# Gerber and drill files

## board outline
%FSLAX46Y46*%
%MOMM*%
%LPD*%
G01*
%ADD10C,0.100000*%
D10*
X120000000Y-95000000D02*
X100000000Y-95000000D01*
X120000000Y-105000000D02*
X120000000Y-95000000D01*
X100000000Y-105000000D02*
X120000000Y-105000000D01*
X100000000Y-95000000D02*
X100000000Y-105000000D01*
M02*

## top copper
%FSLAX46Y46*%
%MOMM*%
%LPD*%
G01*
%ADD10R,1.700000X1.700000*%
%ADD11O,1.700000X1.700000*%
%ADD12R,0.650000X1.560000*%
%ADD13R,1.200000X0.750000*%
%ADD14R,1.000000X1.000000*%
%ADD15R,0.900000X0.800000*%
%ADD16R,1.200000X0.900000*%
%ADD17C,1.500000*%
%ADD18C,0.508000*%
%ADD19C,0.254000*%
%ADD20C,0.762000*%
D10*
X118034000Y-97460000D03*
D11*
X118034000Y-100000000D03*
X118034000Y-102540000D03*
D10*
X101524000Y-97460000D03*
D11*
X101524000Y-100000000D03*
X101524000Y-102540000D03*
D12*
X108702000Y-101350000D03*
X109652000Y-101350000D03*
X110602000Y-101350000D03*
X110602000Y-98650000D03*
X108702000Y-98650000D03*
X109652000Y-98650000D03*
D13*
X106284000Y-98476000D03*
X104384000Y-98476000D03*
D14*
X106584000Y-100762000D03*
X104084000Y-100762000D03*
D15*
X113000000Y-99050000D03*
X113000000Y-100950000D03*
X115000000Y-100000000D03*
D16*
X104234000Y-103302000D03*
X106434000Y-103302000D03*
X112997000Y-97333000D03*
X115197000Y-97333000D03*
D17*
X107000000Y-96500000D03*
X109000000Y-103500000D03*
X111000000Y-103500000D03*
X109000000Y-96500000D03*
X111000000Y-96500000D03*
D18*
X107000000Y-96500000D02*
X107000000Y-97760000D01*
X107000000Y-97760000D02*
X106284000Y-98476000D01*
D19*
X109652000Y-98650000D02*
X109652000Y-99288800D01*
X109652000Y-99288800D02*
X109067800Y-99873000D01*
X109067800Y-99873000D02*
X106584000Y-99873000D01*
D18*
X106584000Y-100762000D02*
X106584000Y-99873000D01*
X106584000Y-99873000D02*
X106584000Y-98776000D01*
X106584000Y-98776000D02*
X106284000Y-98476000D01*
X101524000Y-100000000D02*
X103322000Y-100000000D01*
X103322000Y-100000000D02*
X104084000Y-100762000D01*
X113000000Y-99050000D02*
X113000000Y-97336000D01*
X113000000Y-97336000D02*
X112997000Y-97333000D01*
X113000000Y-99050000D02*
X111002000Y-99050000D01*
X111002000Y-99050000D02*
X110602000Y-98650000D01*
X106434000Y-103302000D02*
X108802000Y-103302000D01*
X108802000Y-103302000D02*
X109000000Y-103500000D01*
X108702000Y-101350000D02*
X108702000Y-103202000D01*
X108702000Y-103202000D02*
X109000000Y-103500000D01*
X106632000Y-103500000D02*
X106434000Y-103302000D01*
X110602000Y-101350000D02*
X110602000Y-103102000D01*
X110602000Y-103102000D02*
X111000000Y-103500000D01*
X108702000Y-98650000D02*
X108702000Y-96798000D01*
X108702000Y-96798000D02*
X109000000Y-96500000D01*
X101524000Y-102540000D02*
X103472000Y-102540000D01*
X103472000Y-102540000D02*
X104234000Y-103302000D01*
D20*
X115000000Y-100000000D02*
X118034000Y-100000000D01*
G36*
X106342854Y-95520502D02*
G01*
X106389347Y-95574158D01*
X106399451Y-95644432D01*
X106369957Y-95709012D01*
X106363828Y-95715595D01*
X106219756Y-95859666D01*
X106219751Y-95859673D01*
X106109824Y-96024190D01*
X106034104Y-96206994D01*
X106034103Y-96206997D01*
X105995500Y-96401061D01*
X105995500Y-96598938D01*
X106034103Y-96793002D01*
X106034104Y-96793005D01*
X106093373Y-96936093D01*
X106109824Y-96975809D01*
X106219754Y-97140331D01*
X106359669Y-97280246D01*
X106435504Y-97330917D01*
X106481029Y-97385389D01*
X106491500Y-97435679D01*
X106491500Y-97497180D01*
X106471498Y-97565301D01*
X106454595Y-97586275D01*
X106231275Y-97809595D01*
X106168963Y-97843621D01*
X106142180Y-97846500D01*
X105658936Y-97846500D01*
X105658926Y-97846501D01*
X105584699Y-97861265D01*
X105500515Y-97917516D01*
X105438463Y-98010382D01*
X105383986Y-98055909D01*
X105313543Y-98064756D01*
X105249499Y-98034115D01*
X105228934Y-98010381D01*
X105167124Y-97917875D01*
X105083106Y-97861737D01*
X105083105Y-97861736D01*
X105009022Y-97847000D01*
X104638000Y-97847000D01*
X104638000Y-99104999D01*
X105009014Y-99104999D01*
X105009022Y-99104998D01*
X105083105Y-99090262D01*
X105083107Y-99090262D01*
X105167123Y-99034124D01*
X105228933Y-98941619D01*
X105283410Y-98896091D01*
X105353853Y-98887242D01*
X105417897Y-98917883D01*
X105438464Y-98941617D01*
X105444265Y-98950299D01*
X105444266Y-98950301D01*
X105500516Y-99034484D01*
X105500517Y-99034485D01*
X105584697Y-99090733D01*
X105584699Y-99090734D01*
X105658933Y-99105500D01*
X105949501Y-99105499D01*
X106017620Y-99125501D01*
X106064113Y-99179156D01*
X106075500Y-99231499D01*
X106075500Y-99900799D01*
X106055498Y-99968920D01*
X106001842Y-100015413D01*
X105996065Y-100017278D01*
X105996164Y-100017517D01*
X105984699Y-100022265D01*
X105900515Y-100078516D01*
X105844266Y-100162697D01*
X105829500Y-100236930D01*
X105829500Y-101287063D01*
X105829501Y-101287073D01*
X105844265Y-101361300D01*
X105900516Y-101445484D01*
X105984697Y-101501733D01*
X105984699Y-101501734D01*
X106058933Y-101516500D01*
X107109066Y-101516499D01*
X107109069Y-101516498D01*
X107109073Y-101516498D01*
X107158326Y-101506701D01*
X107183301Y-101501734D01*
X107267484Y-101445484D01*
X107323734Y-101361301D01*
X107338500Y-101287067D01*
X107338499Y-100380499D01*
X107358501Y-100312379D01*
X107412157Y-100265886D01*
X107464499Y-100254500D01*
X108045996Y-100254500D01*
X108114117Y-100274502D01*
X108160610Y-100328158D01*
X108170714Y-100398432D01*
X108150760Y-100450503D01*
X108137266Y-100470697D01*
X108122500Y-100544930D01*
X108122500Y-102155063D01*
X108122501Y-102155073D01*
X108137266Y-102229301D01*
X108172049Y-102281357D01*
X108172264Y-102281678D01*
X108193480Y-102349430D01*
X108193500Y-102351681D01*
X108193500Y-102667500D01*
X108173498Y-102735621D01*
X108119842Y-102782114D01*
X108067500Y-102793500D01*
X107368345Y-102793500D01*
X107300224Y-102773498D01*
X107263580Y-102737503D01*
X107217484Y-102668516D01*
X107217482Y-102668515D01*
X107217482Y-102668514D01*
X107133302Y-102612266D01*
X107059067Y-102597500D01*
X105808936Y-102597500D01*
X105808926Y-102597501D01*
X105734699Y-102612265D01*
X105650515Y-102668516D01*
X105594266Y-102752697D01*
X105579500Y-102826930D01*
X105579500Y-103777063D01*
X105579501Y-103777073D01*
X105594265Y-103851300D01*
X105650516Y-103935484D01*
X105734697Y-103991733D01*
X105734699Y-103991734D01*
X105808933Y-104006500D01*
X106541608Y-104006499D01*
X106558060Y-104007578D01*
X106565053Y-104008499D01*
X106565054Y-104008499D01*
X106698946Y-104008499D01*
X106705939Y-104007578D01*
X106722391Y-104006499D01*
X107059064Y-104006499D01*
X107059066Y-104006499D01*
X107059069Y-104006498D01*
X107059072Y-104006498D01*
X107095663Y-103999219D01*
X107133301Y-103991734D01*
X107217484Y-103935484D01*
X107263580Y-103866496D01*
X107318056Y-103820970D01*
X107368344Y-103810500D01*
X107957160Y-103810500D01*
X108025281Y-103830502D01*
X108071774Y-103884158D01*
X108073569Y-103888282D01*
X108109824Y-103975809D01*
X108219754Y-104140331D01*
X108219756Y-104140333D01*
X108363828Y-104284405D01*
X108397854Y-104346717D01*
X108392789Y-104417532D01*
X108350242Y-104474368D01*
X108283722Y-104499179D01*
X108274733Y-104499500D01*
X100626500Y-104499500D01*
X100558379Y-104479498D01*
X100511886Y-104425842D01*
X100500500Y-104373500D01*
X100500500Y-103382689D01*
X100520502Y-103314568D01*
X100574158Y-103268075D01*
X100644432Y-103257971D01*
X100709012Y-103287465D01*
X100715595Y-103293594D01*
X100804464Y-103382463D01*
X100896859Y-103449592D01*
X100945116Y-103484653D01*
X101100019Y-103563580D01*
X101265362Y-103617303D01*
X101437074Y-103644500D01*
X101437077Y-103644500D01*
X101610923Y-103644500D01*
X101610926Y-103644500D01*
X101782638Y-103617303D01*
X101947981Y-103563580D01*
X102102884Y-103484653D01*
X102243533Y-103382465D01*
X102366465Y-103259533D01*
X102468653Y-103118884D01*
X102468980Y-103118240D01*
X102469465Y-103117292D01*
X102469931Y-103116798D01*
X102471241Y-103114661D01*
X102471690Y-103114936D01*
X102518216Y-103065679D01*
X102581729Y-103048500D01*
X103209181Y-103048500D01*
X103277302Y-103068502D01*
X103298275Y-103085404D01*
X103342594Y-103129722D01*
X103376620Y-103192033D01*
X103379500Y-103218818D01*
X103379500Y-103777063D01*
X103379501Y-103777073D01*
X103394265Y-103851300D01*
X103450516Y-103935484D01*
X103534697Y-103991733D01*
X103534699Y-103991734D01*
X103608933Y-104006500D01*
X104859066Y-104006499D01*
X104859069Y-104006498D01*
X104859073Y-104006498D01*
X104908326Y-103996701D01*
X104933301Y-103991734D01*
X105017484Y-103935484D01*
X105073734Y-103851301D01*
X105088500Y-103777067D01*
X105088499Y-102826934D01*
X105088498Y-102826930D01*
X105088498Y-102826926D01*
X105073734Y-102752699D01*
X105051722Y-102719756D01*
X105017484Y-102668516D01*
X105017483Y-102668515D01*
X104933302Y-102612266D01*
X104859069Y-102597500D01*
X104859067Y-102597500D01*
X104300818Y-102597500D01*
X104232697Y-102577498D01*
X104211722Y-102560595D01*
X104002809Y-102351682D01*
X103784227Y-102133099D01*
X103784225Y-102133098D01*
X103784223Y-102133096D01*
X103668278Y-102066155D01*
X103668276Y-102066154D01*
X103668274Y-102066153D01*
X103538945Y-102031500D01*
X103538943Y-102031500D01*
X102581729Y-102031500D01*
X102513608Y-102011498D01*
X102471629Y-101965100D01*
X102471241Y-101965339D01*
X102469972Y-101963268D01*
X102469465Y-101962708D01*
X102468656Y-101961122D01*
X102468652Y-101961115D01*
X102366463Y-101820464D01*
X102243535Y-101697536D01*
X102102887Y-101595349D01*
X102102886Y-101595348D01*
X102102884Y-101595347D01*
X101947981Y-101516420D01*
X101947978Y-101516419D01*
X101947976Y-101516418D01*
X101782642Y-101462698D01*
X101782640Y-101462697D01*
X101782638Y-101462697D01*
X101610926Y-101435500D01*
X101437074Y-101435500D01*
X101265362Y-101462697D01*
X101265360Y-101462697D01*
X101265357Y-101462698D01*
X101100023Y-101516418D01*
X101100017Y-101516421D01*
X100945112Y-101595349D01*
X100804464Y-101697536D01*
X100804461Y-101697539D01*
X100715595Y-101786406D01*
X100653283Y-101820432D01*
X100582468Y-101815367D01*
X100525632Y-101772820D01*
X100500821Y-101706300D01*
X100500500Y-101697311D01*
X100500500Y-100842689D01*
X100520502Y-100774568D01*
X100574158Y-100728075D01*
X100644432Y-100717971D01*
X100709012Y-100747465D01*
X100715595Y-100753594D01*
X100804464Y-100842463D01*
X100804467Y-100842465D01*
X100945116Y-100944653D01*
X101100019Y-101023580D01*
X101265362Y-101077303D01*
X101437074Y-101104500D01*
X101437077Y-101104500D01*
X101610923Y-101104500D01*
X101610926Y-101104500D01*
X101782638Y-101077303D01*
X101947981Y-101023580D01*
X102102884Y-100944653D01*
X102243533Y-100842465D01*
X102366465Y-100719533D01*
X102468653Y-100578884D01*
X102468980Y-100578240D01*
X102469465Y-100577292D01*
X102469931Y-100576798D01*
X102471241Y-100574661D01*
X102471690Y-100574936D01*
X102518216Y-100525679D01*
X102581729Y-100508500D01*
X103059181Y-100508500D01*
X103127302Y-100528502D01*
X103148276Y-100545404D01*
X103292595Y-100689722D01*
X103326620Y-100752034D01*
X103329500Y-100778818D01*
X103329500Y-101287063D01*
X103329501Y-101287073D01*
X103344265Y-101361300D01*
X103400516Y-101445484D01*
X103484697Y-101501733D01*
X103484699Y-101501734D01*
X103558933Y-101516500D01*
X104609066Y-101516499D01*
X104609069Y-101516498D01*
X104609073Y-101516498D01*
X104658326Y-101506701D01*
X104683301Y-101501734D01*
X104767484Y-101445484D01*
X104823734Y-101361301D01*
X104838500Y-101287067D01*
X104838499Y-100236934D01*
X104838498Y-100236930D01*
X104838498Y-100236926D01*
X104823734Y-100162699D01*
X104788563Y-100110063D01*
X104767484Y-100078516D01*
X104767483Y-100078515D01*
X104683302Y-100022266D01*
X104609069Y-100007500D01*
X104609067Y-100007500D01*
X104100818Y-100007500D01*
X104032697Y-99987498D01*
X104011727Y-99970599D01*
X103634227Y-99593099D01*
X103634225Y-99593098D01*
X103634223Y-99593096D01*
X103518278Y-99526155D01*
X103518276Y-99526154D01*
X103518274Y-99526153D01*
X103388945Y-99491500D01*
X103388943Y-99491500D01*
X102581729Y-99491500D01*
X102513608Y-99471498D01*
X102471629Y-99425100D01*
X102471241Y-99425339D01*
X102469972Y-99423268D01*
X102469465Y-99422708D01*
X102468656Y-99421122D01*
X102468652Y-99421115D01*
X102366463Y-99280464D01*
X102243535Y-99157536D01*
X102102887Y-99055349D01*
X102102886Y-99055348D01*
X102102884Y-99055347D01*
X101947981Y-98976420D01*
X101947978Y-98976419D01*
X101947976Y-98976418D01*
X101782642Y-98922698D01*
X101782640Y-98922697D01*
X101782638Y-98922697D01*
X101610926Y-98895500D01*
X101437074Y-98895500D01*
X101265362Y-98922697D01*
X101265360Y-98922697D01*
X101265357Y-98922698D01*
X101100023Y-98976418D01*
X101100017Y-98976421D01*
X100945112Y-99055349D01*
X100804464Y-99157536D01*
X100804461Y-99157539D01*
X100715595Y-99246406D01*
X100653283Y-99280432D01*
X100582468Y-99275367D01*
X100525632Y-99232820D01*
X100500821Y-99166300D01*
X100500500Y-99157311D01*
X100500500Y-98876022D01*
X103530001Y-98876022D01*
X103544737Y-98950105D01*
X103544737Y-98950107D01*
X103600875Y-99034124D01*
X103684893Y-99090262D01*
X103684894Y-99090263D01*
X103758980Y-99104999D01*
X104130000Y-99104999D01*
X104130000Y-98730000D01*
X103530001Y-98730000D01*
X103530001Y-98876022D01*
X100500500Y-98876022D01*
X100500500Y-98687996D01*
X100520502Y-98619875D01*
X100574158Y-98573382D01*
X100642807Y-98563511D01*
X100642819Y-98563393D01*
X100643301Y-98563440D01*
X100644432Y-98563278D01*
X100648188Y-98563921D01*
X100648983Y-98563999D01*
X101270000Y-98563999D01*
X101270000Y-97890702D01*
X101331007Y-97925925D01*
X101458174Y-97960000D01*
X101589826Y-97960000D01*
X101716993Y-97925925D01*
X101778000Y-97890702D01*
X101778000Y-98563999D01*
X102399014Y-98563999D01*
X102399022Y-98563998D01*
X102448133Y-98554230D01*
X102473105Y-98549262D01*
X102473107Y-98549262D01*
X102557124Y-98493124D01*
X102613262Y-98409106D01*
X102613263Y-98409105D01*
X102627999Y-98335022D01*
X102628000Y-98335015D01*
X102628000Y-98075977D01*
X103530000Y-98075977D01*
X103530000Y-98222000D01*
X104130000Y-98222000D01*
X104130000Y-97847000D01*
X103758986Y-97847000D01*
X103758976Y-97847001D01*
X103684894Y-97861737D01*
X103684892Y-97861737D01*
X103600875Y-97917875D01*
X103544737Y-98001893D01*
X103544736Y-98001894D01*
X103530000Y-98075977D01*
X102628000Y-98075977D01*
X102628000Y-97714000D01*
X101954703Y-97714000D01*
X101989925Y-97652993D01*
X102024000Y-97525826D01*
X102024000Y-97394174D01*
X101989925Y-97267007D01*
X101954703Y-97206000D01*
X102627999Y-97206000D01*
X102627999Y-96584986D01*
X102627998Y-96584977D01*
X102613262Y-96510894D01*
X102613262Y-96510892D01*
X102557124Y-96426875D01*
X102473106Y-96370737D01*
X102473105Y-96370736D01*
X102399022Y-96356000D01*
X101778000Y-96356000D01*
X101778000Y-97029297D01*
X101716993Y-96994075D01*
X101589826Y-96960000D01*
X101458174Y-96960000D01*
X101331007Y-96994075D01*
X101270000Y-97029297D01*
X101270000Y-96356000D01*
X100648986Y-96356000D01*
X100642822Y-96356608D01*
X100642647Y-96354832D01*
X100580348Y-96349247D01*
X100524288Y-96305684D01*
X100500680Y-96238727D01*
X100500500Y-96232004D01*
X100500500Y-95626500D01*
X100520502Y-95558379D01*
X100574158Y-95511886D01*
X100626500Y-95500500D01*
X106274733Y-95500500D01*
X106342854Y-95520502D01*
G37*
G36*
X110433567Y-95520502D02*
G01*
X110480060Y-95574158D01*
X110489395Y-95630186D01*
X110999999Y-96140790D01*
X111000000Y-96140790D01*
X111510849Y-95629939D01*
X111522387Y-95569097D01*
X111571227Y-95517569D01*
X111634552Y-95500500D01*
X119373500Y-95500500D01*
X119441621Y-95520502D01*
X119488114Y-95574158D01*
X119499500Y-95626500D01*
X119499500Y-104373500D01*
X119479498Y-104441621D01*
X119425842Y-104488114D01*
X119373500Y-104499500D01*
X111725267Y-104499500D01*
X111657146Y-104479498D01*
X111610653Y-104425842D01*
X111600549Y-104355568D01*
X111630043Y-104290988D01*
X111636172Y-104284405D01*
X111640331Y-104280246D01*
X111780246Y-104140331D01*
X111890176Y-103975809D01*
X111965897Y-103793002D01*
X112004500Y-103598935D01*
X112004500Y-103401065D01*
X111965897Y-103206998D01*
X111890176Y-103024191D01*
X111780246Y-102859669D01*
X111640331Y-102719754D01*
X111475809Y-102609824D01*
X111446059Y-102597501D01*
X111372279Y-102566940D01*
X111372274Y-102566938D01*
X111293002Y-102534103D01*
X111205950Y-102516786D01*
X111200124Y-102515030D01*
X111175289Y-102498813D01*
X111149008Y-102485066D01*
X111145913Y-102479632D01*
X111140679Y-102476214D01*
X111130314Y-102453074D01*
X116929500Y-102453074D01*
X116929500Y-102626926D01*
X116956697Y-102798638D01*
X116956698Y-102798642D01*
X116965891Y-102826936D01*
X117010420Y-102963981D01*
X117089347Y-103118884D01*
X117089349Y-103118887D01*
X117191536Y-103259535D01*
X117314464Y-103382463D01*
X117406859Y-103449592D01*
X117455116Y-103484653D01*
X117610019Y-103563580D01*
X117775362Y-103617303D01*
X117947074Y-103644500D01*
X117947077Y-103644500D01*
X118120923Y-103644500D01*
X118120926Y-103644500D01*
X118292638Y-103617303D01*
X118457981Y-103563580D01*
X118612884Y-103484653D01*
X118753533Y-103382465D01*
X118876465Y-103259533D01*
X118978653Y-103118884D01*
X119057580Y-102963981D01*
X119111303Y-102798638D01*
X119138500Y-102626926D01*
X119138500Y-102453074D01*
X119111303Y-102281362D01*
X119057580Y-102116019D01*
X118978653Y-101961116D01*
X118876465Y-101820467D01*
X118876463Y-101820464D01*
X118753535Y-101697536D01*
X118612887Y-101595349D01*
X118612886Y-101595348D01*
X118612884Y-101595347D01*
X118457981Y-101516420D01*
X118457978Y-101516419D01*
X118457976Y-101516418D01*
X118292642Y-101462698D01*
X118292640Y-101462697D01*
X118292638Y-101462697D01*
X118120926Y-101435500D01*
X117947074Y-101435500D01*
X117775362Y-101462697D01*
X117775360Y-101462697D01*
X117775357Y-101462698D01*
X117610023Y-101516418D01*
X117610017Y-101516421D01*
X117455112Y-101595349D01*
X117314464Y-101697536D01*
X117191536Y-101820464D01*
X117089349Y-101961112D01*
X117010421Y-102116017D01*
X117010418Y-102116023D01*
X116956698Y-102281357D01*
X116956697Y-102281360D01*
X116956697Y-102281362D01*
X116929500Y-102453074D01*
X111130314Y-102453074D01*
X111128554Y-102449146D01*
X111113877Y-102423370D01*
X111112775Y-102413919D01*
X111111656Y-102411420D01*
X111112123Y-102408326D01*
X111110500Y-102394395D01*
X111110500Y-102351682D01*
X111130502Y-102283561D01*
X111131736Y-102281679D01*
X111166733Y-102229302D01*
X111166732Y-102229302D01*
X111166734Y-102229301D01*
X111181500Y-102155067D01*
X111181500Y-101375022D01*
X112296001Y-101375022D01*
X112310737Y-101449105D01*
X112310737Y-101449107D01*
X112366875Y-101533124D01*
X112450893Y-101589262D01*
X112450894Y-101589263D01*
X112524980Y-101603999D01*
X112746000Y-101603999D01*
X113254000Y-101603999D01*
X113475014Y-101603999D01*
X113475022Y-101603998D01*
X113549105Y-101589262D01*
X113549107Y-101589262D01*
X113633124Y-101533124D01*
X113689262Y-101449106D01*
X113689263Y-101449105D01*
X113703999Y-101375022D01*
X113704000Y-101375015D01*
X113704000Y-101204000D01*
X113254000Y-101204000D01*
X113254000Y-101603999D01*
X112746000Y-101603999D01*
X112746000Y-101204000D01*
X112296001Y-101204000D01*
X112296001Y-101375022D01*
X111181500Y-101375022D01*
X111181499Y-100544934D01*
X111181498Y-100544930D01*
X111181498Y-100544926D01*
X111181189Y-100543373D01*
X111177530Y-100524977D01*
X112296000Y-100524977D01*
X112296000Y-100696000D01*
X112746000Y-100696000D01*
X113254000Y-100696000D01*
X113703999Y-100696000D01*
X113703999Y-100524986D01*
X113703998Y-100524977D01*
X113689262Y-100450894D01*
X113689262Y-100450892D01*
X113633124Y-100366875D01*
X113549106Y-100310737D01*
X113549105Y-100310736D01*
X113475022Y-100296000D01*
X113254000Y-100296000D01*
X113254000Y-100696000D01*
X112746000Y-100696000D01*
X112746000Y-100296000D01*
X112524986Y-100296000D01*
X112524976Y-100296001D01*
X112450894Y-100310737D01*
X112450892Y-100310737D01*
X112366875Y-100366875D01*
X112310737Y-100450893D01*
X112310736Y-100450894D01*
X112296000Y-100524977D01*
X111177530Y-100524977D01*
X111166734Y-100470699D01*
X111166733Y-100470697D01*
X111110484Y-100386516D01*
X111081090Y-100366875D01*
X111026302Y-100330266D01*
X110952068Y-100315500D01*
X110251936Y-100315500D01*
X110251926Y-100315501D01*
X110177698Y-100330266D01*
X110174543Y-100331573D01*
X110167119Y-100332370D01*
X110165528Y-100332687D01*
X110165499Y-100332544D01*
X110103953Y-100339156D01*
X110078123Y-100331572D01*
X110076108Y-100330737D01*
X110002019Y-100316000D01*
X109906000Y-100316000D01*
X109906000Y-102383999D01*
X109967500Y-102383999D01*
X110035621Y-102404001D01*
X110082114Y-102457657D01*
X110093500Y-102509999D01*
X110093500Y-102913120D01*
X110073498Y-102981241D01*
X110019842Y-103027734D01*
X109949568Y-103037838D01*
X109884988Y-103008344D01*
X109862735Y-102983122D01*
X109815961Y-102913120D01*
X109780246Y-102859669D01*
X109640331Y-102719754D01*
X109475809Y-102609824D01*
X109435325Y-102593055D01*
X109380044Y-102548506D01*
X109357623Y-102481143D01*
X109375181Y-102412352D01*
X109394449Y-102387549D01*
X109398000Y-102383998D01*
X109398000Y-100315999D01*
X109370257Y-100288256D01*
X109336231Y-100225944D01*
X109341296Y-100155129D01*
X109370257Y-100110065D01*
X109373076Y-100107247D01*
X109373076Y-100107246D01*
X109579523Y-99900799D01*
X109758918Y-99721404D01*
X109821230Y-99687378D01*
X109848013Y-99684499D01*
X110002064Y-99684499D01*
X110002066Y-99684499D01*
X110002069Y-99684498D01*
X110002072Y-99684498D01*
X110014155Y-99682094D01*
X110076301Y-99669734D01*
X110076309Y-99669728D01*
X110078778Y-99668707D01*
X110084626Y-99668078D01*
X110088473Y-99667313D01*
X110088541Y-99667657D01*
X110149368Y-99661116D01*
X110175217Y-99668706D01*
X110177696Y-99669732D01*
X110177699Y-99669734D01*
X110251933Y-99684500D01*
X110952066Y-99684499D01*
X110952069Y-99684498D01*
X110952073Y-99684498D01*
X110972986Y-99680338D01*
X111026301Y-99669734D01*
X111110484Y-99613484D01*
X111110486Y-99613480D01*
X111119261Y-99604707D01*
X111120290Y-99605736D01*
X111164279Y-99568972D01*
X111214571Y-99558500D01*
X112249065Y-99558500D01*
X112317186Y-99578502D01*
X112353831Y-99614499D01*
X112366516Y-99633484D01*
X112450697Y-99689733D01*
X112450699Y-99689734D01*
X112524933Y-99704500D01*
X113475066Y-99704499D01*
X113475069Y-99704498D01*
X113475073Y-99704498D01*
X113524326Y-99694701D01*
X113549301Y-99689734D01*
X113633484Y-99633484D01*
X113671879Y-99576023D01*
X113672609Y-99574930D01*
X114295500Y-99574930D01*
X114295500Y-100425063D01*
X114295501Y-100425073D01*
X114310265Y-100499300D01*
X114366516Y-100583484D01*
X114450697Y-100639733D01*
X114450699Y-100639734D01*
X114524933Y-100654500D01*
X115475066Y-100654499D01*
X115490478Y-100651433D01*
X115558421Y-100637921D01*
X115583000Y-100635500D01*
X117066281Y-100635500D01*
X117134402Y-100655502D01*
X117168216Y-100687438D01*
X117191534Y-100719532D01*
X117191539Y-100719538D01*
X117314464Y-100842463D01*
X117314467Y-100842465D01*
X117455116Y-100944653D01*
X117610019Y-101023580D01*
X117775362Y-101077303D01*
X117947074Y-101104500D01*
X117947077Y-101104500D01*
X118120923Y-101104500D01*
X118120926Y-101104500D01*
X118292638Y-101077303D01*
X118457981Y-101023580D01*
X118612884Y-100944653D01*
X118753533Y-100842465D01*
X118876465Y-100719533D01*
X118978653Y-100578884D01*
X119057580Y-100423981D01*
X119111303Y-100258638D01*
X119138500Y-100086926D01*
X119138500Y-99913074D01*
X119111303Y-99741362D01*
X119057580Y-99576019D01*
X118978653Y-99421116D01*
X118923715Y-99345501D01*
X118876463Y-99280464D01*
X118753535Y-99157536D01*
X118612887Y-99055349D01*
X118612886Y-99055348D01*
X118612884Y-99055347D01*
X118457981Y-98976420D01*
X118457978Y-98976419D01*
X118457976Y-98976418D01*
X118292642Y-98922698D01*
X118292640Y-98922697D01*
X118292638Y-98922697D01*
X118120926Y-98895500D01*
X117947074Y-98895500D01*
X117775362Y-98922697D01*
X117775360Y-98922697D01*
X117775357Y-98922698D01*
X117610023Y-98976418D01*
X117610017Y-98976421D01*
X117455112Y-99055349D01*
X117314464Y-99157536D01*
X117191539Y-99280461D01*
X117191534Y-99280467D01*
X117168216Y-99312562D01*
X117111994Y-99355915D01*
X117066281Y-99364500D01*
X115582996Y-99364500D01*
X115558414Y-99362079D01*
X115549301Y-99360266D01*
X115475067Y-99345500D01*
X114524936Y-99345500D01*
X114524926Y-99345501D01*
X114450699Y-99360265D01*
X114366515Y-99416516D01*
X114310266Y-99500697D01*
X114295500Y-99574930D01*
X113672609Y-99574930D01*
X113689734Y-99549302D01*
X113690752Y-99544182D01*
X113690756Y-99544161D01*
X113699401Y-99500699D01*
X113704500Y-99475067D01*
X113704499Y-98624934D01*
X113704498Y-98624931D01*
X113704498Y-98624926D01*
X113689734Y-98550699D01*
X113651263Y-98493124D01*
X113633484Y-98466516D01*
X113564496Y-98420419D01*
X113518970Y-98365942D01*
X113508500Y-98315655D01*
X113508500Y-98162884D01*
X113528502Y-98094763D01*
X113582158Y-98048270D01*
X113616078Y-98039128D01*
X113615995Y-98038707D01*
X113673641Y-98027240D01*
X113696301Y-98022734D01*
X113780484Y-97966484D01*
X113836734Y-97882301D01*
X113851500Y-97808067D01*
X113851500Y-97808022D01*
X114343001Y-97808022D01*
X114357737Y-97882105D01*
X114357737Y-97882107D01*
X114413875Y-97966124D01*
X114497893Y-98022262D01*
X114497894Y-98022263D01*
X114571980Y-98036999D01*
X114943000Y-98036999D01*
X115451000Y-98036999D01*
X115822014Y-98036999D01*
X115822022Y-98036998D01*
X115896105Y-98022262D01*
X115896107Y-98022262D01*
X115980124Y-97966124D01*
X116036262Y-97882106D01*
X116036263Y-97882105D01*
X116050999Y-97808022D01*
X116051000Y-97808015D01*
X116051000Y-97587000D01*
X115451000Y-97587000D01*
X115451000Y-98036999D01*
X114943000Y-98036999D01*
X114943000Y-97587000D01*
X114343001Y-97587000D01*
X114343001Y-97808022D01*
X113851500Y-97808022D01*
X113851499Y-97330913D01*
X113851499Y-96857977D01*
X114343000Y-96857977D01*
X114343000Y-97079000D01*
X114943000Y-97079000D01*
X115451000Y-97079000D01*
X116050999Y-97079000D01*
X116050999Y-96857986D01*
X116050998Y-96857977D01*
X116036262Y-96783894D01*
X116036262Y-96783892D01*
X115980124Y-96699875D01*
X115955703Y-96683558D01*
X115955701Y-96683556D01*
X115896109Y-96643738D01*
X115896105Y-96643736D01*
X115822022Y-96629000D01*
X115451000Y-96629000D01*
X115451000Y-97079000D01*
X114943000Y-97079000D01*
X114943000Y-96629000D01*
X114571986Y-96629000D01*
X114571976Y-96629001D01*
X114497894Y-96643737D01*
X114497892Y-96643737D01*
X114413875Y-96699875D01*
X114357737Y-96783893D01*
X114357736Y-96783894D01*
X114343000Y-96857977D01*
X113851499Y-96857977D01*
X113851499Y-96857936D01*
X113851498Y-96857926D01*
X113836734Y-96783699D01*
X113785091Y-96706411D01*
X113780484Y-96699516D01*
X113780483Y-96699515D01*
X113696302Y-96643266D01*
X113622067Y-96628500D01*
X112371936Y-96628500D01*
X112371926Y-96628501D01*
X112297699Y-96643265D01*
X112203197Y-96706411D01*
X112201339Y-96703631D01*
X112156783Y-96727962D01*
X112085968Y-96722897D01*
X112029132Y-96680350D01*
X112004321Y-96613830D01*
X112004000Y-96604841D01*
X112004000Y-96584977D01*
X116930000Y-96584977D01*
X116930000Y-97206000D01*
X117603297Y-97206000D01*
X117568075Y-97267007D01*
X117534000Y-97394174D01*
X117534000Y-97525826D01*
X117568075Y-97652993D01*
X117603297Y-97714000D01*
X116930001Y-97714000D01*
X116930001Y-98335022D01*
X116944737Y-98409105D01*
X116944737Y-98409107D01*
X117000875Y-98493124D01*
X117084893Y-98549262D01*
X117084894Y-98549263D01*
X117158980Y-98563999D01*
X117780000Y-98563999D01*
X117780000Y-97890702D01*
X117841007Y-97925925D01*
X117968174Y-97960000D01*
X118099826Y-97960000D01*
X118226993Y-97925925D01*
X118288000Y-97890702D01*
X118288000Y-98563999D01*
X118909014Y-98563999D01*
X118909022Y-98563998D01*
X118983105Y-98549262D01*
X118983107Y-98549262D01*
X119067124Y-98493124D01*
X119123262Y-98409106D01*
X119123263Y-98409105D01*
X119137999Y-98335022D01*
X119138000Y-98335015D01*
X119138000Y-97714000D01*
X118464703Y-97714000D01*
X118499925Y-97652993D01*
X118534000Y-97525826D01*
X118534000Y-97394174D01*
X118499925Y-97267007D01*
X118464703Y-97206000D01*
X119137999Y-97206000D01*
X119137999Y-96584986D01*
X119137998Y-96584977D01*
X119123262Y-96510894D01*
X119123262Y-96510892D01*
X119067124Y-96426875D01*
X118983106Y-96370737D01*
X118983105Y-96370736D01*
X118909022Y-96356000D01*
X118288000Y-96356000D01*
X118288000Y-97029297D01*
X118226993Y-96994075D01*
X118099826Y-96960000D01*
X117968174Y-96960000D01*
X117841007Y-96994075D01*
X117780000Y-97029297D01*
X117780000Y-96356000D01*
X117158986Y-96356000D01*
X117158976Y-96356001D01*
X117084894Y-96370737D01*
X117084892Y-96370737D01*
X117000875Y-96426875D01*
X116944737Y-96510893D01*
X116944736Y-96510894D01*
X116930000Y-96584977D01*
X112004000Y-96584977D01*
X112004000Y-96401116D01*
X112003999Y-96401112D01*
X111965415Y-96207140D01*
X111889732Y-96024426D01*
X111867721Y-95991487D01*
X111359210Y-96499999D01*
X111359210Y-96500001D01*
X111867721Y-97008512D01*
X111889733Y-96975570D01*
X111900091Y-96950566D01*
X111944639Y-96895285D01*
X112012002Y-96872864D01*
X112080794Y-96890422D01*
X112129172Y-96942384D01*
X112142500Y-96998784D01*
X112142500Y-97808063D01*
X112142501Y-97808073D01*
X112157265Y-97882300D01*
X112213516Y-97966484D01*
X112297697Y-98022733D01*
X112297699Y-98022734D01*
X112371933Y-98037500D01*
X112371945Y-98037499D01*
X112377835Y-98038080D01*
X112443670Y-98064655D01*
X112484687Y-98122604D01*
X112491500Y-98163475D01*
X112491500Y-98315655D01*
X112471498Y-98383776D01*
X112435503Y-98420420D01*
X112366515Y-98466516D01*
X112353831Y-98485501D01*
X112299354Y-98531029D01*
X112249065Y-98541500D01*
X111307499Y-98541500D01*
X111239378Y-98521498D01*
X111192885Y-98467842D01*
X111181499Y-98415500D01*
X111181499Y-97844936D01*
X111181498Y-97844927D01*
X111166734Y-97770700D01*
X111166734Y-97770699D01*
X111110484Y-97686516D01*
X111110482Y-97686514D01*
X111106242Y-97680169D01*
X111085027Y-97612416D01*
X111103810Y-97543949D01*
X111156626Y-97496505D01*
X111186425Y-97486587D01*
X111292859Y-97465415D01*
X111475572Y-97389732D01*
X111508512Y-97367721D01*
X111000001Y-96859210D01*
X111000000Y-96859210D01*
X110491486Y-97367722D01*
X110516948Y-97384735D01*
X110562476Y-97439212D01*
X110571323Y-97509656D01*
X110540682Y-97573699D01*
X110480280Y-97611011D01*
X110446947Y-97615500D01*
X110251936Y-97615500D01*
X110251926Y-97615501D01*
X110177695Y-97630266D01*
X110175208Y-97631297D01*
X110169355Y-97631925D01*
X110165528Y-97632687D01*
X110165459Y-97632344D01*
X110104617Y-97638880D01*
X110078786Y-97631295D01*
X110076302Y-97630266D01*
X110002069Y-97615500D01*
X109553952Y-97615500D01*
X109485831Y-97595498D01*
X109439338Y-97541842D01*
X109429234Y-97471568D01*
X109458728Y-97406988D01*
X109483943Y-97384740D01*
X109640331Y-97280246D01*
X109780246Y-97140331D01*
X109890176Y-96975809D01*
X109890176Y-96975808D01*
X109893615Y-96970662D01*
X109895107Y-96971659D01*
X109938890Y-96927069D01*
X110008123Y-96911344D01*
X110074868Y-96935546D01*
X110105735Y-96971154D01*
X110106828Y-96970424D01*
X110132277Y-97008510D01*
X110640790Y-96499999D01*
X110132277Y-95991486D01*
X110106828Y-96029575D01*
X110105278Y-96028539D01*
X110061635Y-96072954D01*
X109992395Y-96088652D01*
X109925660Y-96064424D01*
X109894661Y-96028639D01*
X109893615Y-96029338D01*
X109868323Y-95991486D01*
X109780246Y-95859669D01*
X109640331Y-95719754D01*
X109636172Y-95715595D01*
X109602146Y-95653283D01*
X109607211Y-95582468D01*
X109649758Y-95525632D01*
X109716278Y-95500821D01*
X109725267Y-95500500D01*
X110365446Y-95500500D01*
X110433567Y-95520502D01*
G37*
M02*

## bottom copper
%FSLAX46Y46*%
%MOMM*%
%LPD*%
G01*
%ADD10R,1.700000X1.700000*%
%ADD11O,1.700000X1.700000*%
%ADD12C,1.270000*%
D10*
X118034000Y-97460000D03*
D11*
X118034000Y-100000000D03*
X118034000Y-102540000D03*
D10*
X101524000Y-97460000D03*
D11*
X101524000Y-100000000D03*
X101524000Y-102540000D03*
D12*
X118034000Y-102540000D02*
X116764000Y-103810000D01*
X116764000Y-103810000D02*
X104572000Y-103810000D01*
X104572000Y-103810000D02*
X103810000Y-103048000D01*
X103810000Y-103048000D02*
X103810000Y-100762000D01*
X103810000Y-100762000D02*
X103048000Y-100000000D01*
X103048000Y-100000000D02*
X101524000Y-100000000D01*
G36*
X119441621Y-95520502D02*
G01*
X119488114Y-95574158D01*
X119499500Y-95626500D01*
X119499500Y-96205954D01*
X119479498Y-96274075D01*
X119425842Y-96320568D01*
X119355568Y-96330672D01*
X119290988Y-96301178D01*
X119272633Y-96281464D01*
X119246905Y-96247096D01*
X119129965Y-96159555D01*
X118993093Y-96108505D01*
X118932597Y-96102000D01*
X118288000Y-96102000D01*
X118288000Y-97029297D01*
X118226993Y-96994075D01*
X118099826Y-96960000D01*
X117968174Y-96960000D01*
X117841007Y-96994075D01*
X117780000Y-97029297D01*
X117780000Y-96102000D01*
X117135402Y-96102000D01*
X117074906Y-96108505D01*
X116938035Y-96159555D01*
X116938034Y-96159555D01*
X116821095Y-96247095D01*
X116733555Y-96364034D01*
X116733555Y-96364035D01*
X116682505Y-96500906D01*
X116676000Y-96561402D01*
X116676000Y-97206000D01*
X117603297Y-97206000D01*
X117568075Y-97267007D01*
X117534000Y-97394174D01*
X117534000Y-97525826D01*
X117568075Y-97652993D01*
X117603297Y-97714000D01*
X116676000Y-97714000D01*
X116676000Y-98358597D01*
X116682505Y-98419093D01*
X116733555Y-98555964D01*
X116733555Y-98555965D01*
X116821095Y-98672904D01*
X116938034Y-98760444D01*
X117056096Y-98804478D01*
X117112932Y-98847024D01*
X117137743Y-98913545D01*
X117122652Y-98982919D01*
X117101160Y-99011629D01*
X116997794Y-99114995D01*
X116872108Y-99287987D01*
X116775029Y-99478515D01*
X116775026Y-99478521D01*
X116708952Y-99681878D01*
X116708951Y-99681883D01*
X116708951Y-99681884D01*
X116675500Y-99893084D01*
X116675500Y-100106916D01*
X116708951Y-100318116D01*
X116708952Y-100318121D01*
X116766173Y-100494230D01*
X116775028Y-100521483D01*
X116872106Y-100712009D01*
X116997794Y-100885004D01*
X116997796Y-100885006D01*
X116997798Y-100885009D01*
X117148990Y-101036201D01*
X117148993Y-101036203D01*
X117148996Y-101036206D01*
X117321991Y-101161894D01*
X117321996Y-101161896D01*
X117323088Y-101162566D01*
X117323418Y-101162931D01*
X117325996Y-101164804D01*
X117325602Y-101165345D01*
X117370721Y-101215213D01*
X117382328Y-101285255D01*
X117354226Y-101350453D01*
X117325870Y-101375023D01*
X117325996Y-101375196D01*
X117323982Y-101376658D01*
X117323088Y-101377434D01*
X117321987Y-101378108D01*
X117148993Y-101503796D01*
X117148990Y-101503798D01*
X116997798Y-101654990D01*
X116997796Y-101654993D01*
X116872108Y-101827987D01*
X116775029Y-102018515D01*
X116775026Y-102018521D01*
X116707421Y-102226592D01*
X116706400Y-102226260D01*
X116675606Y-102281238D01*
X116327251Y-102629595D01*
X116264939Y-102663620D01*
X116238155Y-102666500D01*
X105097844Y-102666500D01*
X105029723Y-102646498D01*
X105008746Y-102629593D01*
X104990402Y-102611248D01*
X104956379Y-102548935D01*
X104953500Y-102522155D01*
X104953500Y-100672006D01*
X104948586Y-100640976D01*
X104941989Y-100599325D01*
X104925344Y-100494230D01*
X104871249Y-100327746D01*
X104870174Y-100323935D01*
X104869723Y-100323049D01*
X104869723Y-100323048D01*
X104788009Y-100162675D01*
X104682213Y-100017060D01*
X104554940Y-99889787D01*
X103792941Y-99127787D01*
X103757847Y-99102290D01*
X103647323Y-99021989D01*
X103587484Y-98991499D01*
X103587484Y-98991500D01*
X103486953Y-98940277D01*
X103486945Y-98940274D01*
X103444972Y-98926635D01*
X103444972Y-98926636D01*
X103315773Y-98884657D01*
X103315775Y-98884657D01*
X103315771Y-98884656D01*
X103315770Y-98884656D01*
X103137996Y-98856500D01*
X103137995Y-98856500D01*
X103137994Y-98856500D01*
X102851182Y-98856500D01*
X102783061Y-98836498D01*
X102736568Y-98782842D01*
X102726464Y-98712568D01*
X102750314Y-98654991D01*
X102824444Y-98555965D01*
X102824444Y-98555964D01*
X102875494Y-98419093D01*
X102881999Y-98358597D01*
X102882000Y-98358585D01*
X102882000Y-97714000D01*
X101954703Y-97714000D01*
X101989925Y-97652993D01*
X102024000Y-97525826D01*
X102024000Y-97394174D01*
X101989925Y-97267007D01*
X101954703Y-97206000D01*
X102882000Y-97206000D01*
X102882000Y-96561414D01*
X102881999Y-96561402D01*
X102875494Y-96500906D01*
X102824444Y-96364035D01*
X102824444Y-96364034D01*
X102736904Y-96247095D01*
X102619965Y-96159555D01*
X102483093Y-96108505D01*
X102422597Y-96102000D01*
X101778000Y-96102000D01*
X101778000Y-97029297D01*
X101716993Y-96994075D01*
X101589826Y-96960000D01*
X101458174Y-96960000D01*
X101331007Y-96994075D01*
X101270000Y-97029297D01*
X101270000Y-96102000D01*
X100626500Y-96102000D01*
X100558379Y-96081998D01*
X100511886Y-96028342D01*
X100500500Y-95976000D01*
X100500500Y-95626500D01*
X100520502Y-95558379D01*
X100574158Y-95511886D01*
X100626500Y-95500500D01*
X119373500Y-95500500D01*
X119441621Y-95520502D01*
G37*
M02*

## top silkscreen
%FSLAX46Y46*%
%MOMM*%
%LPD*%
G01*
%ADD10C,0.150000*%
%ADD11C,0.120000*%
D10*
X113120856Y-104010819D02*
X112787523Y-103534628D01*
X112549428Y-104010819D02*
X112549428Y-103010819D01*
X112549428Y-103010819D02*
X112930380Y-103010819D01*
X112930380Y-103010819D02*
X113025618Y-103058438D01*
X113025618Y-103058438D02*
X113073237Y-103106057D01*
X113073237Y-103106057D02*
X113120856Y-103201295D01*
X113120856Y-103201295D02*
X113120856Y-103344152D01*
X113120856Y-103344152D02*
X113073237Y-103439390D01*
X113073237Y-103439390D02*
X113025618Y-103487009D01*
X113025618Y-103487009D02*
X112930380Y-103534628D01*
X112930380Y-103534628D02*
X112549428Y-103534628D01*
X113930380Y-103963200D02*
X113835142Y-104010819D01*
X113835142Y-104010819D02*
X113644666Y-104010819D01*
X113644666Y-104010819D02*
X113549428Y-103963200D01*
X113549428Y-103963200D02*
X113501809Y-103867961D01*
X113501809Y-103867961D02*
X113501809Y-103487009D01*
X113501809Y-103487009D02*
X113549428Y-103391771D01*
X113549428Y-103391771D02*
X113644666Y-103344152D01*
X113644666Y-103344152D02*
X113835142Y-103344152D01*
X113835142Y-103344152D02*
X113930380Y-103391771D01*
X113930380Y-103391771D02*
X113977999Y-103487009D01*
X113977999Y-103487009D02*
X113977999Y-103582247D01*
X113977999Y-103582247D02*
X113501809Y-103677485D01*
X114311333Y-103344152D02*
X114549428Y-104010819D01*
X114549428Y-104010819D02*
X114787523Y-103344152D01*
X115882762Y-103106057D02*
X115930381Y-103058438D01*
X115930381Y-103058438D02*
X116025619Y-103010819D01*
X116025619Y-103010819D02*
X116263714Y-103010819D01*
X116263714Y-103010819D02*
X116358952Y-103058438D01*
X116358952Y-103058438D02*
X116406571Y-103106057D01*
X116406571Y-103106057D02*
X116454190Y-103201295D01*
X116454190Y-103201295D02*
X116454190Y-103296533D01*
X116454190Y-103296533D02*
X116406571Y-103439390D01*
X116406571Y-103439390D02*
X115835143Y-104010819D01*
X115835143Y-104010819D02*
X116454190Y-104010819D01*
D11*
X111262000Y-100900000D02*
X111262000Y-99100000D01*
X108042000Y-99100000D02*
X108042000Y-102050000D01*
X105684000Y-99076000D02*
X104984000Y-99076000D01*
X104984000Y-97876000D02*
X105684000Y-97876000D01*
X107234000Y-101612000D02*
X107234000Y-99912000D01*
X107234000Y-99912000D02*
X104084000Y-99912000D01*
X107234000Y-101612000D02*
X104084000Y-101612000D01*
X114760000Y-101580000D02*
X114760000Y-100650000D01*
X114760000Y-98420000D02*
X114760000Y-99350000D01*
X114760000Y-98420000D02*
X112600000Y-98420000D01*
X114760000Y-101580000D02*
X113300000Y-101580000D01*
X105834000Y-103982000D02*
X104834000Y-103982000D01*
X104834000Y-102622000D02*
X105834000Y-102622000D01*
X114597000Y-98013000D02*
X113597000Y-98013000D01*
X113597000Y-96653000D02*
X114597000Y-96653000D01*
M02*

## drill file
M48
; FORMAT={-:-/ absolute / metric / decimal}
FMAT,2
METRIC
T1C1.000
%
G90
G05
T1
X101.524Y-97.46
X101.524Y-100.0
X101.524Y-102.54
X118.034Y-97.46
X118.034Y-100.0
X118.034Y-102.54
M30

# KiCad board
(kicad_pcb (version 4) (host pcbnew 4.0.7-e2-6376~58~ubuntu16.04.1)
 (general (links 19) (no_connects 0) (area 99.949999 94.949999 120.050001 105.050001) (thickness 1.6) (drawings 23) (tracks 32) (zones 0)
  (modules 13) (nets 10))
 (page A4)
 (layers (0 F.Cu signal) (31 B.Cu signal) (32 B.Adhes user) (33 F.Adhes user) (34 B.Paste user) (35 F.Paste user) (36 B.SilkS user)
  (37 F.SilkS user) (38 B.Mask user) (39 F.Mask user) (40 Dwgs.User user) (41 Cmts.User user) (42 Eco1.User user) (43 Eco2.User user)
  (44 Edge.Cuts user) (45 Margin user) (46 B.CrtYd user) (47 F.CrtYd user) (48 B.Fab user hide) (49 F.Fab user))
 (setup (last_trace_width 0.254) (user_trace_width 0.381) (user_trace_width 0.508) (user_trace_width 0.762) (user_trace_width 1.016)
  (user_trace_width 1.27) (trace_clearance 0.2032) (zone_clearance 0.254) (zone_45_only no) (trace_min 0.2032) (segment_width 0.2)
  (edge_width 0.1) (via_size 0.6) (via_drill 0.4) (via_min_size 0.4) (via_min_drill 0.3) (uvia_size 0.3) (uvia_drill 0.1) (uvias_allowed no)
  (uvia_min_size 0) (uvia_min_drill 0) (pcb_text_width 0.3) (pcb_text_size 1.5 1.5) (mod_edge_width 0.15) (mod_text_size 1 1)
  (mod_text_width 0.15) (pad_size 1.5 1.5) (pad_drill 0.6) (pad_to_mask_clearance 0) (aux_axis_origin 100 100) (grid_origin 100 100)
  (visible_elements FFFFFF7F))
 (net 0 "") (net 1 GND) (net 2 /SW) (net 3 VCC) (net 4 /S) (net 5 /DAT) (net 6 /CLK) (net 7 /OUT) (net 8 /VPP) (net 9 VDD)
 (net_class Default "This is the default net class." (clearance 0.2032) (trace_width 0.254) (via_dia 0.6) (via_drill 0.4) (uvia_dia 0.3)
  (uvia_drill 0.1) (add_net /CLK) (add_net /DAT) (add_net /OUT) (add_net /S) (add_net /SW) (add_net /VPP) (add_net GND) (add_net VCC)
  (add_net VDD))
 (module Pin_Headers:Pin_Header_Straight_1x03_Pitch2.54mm (layer B.Cu) (at 118.034 97.46 180)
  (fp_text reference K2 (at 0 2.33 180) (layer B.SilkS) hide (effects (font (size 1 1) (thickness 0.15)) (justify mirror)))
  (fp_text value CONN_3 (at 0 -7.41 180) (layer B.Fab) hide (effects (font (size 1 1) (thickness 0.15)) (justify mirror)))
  (pad 1 thru_hole rect (at 0 0 180) (size 1.7 1.7) (drill 1) (layers *.Cu *.Mask) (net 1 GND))
  (pad 2 thru_hole oval (at 0 -2.54 180) (size 1.7 1.7) (drill 1) (layers *.Cu *.Mask) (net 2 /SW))
  (pad 3 thru_hole oval (at 0 -5.08 180) (size 1.7 1.7) (drill 1) (layers *.Cu *.Mask) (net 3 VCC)))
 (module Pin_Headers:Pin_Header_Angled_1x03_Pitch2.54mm (layer B.Cu) (at 101.524 97.46 180)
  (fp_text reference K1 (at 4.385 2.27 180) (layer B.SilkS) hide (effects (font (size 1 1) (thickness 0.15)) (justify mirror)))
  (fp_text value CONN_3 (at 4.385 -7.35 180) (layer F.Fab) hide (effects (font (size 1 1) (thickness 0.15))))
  (pad 1 thru_hole rect (at 0 0 180) (size 1.7 1.7) (drill 1) (layers *.Cu *.Mask) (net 1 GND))
  (pad 2 thru_hole oval (at 0 -2.54 180) (size 1.7 1.7) (drill 1) (layers *.Cu *.Mask) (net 3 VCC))
  (pad 3 thru_hole oval (at 0 -5.08 180) (size 1.7 1.7) (drill 1) (layers *.Cu *.Mask) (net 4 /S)))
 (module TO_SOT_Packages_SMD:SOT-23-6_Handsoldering (layer F.Cu) (at 109.652 100 90)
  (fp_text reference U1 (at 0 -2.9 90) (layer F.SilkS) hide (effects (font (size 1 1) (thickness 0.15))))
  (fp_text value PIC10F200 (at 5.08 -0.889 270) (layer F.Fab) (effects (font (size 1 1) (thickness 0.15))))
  (fp_line (start -0.9 1.61) (end 0.9 1.61) (layer F.SilkS) (width 0.12))
  (fp_line (start 0.9 -1.61) (end -2.05 -1.61) (layer F.SilkS) (width 0.12))
  (pad 1 smd rect (at -1.35 -0.95 90) (size 1.56 0.65) (layers F.Cu F.Paste F.Mask) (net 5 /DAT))
  (pad 2 smd rect (at -1.35 0 90) (size 1.56 0.65) (layers F.Cu F.Paste F.Mask) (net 1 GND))
  (pad 3 smd rect (at -1.35 0.95 90) (size 1.56 0.65) (layers F.Cu F.Paste F.Mask) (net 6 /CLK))
  (pad 4 smd rect (at 1.35 0.95 90) (size 1.56 0.65) (layers F.Cu F.Paste F.Mask) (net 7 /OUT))
  (pad 6 smd rect (at 1.35 -0.95 90) (size 1.56 0.65) (layers F.Cu F.Paste F.Mask) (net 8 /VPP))
  (pad 5 smd rect (at 1.35 0 90) (size 1.56 0.65) (layers F.Cu F.Paste F.Mask) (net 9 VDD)))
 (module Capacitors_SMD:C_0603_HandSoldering (layer F.Cu) (at 105.334 98.476 180)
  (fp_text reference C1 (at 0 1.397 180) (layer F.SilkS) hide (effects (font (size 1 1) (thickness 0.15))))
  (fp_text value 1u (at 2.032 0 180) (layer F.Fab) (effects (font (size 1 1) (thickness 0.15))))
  (fp_line (start -0.35 -0.6) (end 0.35 -0.6) (layer F.SilkS) (width 0.12))
  (fp_line (start 0.35 0.6) (end -0.35 0.6) (layer F.SilkS) (width 0.12))
  (pad 1 smd rect (at -0.95 0 180) (size 1.2 0.75) (layers F.Cu F.Paste F.Mask) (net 9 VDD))
  (pad 2 smd rect (at 0.95 0 180) (size 1.2 0.75) (layers F.Cu F.Paste F.Mask) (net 1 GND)))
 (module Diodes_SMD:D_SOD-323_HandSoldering (layer F.Cu) (at 105.334 100.762 180)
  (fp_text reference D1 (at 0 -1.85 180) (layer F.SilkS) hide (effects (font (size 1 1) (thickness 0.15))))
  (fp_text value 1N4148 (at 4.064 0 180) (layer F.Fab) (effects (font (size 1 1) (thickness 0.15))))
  (fp_line (start -1.9 -0.85) (end -1.9 0.85) (layer F.SilkS) (width 0.12))
  (fp_line (start -1.9 0.85) (end 1.25 0.85) (layer F.SilkS) (width 0.12))
  (fp_line (start -1.9 -0.85) (end 1.25 -0.85) (layer F.SilkS) (width 0.12))
  (pad 1 smd rect (at -1.25 0 180) (size 1 1) (layers F.Cu F.Paste F.Mask) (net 9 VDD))
  (pad 2 smd rect (at 1.25 0 180) (size 1 1) (layers F.Cu F.Paste F.Mask) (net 3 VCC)))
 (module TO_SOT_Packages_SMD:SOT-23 (layer F.Cu) (at 114 100)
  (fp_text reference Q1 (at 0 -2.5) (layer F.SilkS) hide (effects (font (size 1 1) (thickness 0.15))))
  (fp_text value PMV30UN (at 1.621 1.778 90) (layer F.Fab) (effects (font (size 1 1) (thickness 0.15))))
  (fp_line (start 0.76 1.58) (end 0.76 0.65) (layer F.SilkS) (width 0.12))
  (fp_line (start 0.76 -1.58) (end 0.76 -0.65) (layer F.SilkS) (width 0.12))
  (fp_line (start 0.76 -1.58) (end -1.4 -1.58) (layer F.SilkS) (width 0.12))
  (fp_line (start 0.76 1.58) (end -0.7 1.58) (layer F.SilkS) (width 0.12))
  (pad 1 smd rect (at -1 -0.95) (size 0.9 0.8) (layers F.Cu F.Paste F.Mask) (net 7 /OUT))
  (pad 2 smd rect (at -1 0.95) (size 0.9 0.8) (layers F.Cu F.Paste F.Mask) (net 1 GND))
  (pad 3 smd rect (at 1 0) (size 0.9 0.8) (layers F.Cu F.Paste F.Mask) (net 2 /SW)))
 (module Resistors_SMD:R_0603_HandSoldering (layer F.Cu) (at 105.334 103.302)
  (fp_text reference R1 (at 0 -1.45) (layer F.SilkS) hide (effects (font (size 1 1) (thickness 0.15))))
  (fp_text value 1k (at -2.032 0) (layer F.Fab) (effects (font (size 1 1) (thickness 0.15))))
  (fp_line (start 0.5 0.68) (end -0.5 0.68) (layer F.SilkS) (width 0.12))
  (fp_line (start -0.5 -0.68) (end 0.5 -0.68) (layer F.SilkS) (width 0.12))
  (pad 1 smd rect (at -1.1 0) (size 1.2 0.9) (layers F.Cu F.Paste F.Mask) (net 4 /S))
  (pad 2 smd rect (at 1.1 0) (size 1.2 0.9) (layers F.Cu F.Paste F.Mask) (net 5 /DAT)))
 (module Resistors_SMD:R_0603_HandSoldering (layer F.Cu) (at 114.097 97.333)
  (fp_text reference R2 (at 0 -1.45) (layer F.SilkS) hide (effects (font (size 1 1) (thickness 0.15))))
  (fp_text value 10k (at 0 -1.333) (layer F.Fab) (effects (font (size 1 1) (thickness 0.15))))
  (fp_line (start 0.5 0.68) (end -0.5 0.68) (layer F.SilkS) (width 0.12))
  (fp_line (start -0.5 -0.68) (end 0.5 -0.68) (layer F.SilkS) (width 0.12))
  (pad 1 smd rect (at -1.1 0) (size 1.2 0.9) (layers F.Cu F.Paste F.Mask) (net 7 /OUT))
  (pad 2 smd rect (at 1.1 0) (size 1.2 0.9) (layers F.Cu F.Paste F.Mask) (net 1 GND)))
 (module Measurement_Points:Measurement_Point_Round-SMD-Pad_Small (layer F.Cu) (at 107 96.5)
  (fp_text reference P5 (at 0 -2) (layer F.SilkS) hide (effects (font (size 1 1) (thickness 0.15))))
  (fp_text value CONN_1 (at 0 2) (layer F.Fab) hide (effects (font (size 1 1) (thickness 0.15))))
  (pad 1 smd circle (at 0 0) (size 1.5 1.5) (layers F.Cu F.Mask) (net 9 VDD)))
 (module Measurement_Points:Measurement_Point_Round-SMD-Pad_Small (layer F.Cu) (at 109 103.5)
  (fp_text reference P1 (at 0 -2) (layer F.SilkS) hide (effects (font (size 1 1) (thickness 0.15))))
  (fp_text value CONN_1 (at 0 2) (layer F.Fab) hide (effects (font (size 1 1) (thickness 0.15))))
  (pad 1 smd circle (at 0 0) (size 1.5 1.5) (layers F.Cu F.Mask) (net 5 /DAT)))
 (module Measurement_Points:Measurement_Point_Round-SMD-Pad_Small (layer F.Cu) (at 111 103.5)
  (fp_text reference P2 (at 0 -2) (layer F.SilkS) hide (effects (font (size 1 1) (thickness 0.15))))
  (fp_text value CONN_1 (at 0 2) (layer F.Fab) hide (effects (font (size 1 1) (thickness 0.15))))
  (pad 1 smd circle (at 0 0) (size 1.5 1.5) (layers F.Cu F.Mask) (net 6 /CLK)))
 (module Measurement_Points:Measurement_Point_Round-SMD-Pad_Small (layer F.Cu) (at 109 96.5)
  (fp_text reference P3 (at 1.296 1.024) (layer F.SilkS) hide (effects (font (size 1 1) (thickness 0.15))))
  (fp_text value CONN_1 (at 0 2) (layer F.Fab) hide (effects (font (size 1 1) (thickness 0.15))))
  (pad 1 smd circle (at 0 0) (size 1.5 1.5) (layers F.Cu F.Mask) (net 8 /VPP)))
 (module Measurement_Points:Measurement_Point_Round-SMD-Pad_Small (layer F.Cu) (at 111 96.5)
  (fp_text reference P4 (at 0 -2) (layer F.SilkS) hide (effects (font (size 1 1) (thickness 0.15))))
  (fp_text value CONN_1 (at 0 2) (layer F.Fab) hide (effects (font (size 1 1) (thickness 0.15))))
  (pad 1 smd circle (at 0 0) (size 1.5 1.5) (layers F.Cu F.Mask) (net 1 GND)))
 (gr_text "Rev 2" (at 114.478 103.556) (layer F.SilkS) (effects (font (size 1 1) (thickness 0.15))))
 (gr_line (start 120 95) (end 100 95) (layer Edge.Cuts) (width 0.1))
 (gr_line (start 120 105) (end 120 95) (layer Edge.Cuts) (width 0.1))
 (gr_line (start 100 105) (end 120 105) (layer Edge.Cuts) (width 0.1))
 (gr_line (start 100 95) (end 100 105) (layer Edge.Cuts) (width 0.1))
 (segment (start 107 96.5) (end 107 97.76) (width 0.508) (layer F.Cu) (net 9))
 (segment (start 107 97.76) (end 106.284 98.476) (width 0.508) (layer F.Cu) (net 9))
 (segment (start 109.652 98.65) (end 109.652 99.2888) (width 0.254) (layer F.Cu) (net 9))
 (segment (start 109.652 99.2888) (end 109.0678 99.873) (width 0.254) (layer F.Cu) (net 9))
 (segment (start 109.0678 99.873) (end 106.584 99.873) (width 0.254) (layer F.Cu) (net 9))
 (segment (start 106.584 100.762) (end 106.584 99.873) (width 0.508) (layer F.Cu) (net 9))
 (segment (start 106.584 99.873) (end 106.584 98.776) (width 0.508) (layer F.Cu) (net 9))
 (segment (start 106.584 98.776) (end 106.284 98.476) (width 0.508) (layer F.Cu) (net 9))
 (segment (start 118.034 102.54) (end 116.764 103.81) (width 1.27) (layer B.Cu) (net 3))
 (segment (start 116.764 103.81) (end 104.572 103.81) (width 1.27) (layer B.Cu) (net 3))
 (segment (start 104.572 103.81) (end 103.81 103.048) (width 1.27) (layer B.Cu) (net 3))
 (segment (start 103.81 103.048) (end 103.81 100.762) (width 1.27) (layer B.Cu) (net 3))
 (segment (start 103.81 100.762) (end 103.048 100) (width 1.27) (layer B.Cu) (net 3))
 (segment (start 103.048 100) (end 101.524 100) (width 1.27) (layer B.Cu) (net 3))
 (segment (start 101.524 100) (end 103.322 100) (width 0.508) (layer F.Cu) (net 3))
 (segment (start 103.322 100) (end 104.084 100.762) (width 0.508) (layer F.Cu) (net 3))
 (segment (start 113 99.05) (end 113 97.336) (width 0.508) (layer F.Cu) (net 7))
 (segment (start 113 97.336) (end 112.997 97.333) (width 0.508) (layer F.Cu) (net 7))
 (segment (start 113 99.05) (end 111.002 99.05) (width 0.508) (layer F.Cu) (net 7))
 (segment (start 111.002 99.05) (end 110.602 98.65) (width 0.508) (layer F.Cu) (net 7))
 (segment (start 106.434 103.302) (end 108.802 103.302) (width 0.508) (layer F.Cu) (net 5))
 (segment (start 108.802 103.302) (end 109 103.5) (width 0.508) (layer F.Cu) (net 5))
 (segment (start 108.702 101.35) (end 108.702 103.202) (width 0.508) (layer F.Cu) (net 5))
 (segment (start 108.702 103.202) (end 109 103.5) (width 0.508) (layer F.Cu) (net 5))
 (segment (start 106.632 103.5) (end 106.434 103.302) (width 0.508) (layer F.Cu) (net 5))
 (segment (start 110.602 101.35) (end 110.602 103.102) (width 0.508) (layer F.Cu) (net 6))
 (segment (start 110.602 103.102) (end 111 103.5) (width 0.508) (layer F.Cu) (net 6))
 (segment (start 108.702 98.65) (end 108.702 96.798) (width 0.508) (layer F.Cu) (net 8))
 (segment (start 108.702 96.798) (end 109 96.5) (width 0.508) (layer F.Cu) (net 8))
 (segment (start 101.524 102.54) (end 103.472 102.54) (width 0.508) (layer F.Cu) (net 4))
 (segment (start 103.472 102.54) (end 104.234 103.302) (width 0.508) (layer F.Cu) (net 4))
 (segment (start 115 100) (end 118.034 100) (width 0.762) (layer F.Cu) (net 2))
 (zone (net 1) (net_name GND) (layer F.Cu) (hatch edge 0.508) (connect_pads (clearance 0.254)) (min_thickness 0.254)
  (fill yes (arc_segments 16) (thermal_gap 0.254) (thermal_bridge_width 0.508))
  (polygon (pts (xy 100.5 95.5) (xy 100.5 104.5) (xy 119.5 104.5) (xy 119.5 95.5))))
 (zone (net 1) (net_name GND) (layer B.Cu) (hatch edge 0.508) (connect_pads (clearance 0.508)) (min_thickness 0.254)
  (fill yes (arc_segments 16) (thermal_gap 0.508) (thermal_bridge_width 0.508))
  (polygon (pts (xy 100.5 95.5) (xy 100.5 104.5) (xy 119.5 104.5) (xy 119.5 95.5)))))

